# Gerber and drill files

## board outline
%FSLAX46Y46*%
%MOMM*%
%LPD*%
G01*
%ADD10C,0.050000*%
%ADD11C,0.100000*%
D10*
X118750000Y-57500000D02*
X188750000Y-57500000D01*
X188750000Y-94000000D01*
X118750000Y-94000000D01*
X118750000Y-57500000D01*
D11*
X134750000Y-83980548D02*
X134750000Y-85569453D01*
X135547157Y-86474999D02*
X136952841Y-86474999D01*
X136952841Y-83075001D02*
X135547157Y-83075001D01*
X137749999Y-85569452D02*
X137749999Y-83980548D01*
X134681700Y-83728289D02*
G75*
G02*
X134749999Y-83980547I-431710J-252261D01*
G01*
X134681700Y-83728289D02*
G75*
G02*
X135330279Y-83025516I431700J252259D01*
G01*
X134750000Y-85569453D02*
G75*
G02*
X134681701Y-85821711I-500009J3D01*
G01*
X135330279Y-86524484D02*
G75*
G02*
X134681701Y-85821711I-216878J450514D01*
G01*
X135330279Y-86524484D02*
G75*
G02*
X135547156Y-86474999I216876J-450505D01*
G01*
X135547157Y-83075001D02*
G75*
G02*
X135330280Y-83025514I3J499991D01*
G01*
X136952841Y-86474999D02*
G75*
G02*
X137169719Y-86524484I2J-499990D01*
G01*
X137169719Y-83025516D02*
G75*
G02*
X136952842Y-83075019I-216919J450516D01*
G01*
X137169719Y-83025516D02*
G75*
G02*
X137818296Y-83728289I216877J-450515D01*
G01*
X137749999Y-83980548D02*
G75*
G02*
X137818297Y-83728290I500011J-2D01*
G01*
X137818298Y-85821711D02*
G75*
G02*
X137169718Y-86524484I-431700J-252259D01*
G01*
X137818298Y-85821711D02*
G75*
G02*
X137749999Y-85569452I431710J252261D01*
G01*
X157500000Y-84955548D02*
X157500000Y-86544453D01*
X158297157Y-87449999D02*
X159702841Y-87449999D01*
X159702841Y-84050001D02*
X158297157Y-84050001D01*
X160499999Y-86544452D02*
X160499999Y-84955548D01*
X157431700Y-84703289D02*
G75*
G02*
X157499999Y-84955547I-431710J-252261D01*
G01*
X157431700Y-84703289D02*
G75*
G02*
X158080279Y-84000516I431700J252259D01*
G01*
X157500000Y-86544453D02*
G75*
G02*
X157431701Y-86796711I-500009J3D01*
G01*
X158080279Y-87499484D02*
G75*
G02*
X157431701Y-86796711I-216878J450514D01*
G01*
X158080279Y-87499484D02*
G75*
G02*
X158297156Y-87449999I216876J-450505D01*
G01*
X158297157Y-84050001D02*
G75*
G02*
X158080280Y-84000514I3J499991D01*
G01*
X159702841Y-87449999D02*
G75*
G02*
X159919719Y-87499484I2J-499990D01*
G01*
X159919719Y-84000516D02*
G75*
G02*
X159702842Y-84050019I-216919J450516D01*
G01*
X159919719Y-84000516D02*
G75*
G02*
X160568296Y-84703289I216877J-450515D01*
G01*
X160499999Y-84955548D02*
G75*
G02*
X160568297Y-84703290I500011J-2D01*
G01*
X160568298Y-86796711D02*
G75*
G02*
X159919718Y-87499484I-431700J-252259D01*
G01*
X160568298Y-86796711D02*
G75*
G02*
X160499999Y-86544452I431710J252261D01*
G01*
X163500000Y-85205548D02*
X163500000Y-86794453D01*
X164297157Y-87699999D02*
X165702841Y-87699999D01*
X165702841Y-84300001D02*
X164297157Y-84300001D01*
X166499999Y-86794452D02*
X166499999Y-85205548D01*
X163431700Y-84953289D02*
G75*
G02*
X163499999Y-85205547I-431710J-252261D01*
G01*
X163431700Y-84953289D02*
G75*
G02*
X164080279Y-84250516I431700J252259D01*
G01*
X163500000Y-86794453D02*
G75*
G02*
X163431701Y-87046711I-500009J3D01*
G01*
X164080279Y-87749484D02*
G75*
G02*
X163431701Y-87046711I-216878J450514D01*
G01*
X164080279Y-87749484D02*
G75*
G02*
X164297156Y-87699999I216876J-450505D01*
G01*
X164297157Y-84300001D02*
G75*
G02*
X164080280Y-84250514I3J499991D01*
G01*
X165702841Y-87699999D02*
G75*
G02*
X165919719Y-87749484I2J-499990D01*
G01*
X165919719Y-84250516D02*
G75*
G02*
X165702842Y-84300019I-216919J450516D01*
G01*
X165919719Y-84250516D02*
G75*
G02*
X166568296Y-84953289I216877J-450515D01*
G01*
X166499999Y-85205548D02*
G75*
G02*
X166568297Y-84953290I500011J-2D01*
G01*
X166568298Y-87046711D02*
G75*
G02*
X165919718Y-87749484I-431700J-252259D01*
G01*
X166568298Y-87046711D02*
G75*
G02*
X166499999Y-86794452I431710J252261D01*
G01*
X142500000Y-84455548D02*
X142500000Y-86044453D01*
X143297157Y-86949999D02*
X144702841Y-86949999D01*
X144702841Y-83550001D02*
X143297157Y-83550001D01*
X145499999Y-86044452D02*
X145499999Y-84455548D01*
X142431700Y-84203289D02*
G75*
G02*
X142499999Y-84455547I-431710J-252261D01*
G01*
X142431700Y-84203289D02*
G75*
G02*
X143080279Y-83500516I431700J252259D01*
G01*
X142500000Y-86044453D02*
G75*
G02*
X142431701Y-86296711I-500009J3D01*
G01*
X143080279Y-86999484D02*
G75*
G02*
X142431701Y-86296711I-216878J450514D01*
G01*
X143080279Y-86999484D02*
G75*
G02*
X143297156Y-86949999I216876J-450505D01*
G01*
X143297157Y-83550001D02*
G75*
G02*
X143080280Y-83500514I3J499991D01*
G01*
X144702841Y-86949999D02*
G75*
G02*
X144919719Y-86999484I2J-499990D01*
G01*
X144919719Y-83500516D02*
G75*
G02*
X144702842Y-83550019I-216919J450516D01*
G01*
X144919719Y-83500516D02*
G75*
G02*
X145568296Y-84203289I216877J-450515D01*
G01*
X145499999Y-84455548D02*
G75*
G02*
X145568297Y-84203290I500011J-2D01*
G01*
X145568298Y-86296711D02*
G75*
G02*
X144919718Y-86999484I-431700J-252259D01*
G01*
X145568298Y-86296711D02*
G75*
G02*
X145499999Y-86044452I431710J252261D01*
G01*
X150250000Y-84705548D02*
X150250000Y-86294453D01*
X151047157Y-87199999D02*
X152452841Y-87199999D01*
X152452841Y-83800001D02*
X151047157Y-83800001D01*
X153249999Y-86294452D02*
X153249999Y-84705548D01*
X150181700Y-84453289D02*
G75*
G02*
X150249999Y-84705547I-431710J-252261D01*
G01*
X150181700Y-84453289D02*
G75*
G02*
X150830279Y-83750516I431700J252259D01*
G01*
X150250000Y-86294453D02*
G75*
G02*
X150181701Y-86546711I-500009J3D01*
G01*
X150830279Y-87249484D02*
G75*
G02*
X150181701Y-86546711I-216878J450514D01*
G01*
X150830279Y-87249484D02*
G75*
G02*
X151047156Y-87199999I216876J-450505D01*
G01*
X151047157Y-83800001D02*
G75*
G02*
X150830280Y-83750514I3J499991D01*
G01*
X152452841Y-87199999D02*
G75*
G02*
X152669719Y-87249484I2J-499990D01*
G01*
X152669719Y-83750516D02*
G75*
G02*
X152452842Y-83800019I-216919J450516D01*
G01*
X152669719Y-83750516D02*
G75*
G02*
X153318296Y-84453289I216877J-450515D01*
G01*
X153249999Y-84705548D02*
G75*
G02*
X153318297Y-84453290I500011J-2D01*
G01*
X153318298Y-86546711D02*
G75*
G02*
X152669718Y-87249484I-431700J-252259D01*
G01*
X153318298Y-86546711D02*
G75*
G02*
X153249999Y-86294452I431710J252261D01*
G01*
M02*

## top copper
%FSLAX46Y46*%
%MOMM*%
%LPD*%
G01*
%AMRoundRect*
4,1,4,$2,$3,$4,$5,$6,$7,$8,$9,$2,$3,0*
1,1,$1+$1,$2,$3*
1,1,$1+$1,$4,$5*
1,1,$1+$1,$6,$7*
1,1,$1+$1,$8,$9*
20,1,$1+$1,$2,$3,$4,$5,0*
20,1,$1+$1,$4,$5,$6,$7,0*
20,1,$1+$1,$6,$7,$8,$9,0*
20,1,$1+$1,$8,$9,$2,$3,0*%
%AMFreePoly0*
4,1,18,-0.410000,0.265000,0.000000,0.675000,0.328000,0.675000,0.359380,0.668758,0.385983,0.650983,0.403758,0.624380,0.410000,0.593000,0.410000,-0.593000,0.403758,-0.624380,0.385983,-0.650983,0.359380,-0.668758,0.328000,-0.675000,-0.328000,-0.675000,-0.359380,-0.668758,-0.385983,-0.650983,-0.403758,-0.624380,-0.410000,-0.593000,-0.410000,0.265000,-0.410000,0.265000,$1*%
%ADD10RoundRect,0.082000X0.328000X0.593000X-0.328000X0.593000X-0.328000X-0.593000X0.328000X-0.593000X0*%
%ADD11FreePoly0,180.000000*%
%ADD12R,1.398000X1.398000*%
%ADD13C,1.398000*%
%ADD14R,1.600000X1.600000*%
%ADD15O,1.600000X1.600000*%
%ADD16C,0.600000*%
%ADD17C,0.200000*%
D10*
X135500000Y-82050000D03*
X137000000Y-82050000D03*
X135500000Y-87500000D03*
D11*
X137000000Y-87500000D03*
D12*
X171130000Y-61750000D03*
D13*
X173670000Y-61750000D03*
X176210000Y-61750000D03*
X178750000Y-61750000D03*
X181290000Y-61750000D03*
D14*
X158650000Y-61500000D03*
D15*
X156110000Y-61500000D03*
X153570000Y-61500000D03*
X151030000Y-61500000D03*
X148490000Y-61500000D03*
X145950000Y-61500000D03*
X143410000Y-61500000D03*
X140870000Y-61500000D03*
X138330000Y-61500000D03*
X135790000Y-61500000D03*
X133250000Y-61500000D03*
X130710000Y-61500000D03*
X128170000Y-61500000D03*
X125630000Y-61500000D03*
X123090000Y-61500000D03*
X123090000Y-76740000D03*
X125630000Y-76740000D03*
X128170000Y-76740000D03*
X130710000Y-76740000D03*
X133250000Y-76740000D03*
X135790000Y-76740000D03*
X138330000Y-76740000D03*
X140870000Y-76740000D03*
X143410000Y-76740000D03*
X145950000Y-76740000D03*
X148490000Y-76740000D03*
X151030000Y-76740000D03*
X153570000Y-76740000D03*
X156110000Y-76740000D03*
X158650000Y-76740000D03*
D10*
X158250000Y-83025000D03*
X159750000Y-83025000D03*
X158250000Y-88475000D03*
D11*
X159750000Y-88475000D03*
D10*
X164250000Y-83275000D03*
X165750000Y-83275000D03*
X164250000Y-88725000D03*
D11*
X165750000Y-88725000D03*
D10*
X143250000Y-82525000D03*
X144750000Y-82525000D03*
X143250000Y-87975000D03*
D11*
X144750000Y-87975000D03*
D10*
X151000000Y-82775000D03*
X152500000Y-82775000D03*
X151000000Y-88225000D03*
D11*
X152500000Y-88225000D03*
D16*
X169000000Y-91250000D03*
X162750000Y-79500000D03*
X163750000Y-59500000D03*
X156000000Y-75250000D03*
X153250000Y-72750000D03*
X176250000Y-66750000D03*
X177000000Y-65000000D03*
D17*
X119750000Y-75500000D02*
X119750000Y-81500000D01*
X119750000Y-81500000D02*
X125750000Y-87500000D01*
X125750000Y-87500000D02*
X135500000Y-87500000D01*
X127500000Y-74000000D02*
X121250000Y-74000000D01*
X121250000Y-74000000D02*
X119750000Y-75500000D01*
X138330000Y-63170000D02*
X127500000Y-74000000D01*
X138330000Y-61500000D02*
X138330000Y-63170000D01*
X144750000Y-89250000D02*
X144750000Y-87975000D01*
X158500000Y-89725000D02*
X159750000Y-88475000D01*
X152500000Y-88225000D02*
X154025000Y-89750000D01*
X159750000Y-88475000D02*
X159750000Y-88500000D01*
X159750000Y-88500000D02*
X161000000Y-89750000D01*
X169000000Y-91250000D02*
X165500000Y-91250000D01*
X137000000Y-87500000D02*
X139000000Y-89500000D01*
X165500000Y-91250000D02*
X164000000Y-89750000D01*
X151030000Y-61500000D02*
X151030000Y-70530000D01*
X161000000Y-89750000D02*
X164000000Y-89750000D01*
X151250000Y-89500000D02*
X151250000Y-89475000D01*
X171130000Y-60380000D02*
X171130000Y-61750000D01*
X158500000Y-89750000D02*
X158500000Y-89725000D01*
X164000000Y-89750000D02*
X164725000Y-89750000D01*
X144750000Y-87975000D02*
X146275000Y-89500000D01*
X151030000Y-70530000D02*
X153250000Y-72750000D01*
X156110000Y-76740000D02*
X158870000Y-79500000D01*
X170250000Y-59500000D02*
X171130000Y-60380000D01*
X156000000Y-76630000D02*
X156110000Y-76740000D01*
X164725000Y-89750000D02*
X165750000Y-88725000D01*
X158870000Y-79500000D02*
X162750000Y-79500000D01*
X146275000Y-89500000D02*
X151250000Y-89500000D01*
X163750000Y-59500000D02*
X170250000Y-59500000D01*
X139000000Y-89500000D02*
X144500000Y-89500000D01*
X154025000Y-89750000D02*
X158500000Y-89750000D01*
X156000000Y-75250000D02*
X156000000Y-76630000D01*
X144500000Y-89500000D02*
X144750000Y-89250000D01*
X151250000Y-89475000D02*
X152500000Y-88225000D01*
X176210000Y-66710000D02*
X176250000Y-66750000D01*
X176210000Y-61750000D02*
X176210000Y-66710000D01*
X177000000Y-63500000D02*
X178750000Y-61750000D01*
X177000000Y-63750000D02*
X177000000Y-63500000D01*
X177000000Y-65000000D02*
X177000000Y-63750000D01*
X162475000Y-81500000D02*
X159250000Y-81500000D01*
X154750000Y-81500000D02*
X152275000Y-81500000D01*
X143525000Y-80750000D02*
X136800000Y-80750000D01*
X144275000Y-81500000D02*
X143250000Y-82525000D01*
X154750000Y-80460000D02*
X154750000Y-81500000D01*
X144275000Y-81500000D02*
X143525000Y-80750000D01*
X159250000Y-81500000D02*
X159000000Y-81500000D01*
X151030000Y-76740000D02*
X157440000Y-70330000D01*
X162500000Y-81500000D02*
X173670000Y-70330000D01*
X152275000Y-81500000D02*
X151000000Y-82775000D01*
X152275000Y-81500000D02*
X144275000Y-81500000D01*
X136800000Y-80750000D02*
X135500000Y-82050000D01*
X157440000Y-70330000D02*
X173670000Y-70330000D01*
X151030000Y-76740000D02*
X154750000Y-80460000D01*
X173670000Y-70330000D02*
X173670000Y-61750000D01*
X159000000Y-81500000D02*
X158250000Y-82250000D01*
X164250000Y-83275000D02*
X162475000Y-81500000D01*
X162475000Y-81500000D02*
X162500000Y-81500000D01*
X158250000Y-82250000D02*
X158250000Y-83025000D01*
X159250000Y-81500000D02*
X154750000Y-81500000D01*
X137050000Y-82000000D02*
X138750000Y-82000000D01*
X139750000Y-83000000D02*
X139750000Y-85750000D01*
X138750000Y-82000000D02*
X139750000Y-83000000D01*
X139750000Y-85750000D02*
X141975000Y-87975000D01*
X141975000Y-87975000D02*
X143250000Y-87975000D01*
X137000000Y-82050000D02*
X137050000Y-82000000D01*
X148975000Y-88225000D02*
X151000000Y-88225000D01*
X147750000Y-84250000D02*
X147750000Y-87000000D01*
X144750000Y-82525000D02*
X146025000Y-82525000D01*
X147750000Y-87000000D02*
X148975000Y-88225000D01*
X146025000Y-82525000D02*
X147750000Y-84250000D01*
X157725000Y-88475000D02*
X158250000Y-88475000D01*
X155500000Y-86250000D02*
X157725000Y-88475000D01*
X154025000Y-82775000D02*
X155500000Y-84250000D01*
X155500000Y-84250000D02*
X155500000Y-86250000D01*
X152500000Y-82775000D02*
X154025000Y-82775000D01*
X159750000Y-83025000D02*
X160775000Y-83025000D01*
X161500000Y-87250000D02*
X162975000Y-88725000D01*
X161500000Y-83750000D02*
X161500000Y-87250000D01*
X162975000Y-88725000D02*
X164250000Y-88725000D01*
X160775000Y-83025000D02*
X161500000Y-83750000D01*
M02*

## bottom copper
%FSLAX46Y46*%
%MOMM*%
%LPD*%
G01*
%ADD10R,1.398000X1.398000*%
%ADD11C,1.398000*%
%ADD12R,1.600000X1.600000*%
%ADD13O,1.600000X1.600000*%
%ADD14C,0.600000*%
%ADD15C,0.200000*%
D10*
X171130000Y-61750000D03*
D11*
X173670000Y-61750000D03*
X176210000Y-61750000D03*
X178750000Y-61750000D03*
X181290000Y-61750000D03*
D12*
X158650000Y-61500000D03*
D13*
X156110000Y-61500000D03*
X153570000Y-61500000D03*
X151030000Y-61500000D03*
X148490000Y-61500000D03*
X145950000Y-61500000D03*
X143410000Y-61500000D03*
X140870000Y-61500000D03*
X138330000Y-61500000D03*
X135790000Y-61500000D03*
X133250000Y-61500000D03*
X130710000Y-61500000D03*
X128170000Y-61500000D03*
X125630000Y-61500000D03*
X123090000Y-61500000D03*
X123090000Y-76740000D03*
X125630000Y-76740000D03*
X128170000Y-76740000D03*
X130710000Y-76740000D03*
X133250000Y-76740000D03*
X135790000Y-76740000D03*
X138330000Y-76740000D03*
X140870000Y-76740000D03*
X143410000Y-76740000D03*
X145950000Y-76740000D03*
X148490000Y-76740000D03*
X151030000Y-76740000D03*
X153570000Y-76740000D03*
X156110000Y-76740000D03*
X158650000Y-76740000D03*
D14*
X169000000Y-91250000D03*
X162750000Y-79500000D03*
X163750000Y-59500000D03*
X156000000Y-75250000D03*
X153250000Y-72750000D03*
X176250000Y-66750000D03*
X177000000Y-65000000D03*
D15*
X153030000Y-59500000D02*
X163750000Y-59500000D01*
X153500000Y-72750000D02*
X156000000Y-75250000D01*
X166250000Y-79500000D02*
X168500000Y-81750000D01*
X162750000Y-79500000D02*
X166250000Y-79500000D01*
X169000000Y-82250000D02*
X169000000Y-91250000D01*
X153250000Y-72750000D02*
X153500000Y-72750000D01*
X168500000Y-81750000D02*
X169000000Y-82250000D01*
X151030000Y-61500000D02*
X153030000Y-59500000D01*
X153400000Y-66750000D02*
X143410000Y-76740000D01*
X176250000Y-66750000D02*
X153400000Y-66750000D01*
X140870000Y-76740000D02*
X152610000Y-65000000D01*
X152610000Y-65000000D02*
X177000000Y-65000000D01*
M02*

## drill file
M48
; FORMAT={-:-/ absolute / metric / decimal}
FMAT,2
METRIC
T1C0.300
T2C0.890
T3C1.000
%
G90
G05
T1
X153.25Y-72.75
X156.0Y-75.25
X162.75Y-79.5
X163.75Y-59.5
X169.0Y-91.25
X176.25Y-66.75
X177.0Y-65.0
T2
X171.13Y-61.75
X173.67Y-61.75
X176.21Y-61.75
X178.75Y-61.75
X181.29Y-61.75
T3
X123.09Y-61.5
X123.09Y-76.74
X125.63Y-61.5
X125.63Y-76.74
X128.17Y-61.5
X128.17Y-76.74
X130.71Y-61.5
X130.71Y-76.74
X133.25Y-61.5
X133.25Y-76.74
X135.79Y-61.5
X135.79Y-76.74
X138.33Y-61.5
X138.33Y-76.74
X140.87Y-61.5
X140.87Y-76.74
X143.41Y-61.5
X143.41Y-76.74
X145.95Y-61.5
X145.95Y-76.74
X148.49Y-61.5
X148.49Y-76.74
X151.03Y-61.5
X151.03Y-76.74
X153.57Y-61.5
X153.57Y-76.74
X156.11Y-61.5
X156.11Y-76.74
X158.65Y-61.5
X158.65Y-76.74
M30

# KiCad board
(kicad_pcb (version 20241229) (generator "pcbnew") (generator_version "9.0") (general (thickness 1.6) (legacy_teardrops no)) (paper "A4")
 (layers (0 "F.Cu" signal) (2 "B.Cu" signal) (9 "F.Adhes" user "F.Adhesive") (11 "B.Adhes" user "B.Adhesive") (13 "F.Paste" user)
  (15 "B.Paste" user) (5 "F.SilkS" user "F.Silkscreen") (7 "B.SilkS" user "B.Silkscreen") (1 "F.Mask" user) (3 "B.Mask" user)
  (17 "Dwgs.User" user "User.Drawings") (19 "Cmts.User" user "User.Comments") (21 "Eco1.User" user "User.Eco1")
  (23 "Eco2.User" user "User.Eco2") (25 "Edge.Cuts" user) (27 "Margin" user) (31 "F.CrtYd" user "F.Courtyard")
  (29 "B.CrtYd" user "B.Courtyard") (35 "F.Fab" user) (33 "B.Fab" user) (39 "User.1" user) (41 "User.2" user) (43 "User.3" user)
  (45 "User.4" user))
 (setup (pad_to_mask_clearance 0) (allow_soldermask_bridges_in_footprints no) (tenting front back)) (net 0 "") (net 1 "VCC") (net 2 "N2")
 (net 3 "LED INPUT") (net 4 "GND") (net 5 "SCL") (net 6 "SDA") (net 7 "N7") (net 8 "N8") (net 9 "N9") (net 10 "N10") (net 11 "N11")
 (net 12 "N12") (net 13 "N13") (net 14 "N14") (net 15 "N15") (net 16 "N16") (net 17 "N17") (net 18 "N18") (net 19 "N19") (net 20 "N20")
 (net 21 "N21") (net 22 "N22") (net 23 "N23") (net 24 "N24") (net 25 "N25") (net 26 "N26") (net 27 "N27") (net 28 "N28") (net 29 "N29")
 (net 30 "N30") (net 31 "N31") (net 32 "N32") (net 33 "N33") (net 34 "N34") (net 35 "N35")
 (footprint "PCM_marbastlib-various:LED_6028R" (layer "F.Cu") (at 136.25 84.775 90)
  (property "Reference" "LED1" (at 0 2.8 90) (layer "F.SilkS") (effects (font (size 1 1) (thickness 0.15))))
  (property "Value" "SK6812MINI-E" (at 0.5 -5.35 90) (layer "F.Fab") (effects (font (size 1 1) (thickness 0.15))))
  (fp_line (start 0.794452 -1.5) (end -0.794453 -1.5) (stroke (width 0.1) (type solid)) (layer "Edge.Cuts"))
  (fp_line (start -1.699999 -0.702843) (end -1.699999 0.702841) (stroke (width 0.1) (type solid)) (layer "Edge.Cuts"))
  (fp_line (start 1.699999 0.702841) (end 1.699999 -0.702843) (stroke (width 0.1) (type solid)) (layer "Edge.Cuts"))
  (fp_line (start -0.794452 1.499999) (end 0.794452 1.499999) (stroke (width 0.1) (type solid)) (layer "Edge.Cuts"))
  (fp_arc (start 1.046711 -1.5683) (mid 0.925123 -1.517378) (end 0.794453 -1.500001) (stroke (width 0.1) (type solid)) (layer "Edge.Cuts"))
  (fp_arc (start 1.046711 -1.5683) (mid 1.638071 -1.504036) (end 1.749484 -0.919721) (stroke (width 0.1) (type solid)) (layer "Edge.Cuts"))
  (fp_arc (start -0.794453 -1.5) (mid -0.925123 -1.517377) (end -1.046711 -1.568299) (stroke (width 0.1) (type solid)) (layer "Edge.Cuts"))
  (fp_arc (start -1.749484 -0.919721) (mid -1.638071 -1.504036) (end -1.046711 -1.568299) (stroke (width 0.1) (type solid))
   (layer "Edge.Cuts"))
  (fp_arc (start -1.749484 -0.919721) (mid -1.712527 -0.814069) (end -1.699999 -0.702844) (stroke (width 0.1) (type solid))
   (layer "Edge.Cuts"))
  (fp_arc (start 1.699999 -0.702843) (mid 1.712527 -0.814069) (end 1.749484 -0.919721) (stroke (width 0.1) (type solid)) (layer "Edge.Cuts"))
  (fp_arc (start -1.699999 0.702841) (mid -1.712527 0.814067) (end -1.749484 0.919719) (stroke (width 0.1) (type solid)) (layer "Edge.Cuts"))
  (fp_arc (start 1.749484 0.919719) (mid 1.712527 0.814067) (end 1.699999 0.702842) (stroke (width 0.1) (type solid)) (layer "Edge.Cuts"))
  (fp_arc (start 1.749484 0.919719) (mid 1.63807 1.504033) (end 1.046711 1.568296) (stroke (width 0.1) (type solid)) (layer "Edge.Cuts"))
  (fp_arc (start 0.794452 1.499999) (mid 0.925122 1.517376) (end 1.04671 1.568298) (stroke (width 0.1) (type solid)) (layer "Edge.Cuts"))
  (fp_arc (start -1.046711 1.568298) (mid -1.638072 1.504034) (end -1.749484 0.919718) (stroke (width 0.1) (type solid)) (layer "Edge.Cuts"))
  (fp_arc (start -1.046711 1.568298) (mid -0.925123 1.517376) (end -0.794452 1.499999) (stroke (width 0.1) (type solid)) (layer "Edge.Cuts"))
  (pad "1" smd roundrect (at 2.725 -0.75 180) (size 0.82 1.35) (layers "F.Cu" "F.Mask" "F.Paste") (roundrect_rratio 0.1) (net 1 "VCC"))
  (pad "2" smd roundrect (at 2.725 0.75 180) (size 0.82 1.35) (layers "F.Cu" "F.Mask" "F.Paste") (roundrect_rratio 0.1) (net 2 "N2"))
  (pad "3" smd roundrect (at -2.725 -0.75 180) (size 0.82 1.35) (layers "F.Cu" "F.Mask" "F.Paste") (roundrect_rratio 0.1)
   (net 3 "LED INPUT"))
  (pad "4" smd roundrect (at -2.725 0.75 180) (size 0.82 1.35) (layers "F.Cu" "F.Mask" "F.Paste") (roundrect_rratio 0.1) (chamfer_ratio 0.5)
   (chamfer top_left) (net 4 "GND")))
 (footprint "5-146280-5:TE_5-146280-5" (layer "F.Cu") (at 176.21 61.75)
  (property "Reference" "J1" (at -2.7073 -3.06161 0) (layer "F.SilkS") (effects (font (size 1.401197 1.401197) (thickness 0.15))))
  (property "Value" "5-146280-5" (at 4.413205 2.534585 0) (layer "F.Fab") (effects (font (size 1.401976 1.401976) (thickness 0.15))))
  (pad "1" thru_hole rect (at -5.08 0) (size 1.398 1.398) (drill 0.89) (layers "*.Cu" "*.Mask") (remove_unused_layers no) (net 4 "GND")
   (solder_mask_margin 0.102))
  (pad "2" thru_hole circle (at -2.54 0) (size 1.398 1.398) (drill 0.89) (layers "*.Cu" "*.Mask") (remove_unused_layers no) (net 1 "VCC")
   (solder_mask_margin 0.102))
  (pad "3" thru_hole circle (at 0 0) (size 1.398 1.398) (drill 0.89) (layers "*.Cu" "*.Mask") (remove_unused_layers no) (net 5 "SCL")
   (solder_mask_margin 0.102))
  (pad "4" thru_hole circle (at 2.54 0) (size 1.398 1.398) (drill 0.89) (layers "*.Cu" "*.Mask") (remove_unused_layers no) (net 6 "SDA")
   (solder_mask_margin 0.102))
  (pad "5" thru_hole circle (at 5.08 0) (size 1.398 1.398) (drill 0.89) (layers "*.Cu" "*.Mask") (remove_unused_layers no) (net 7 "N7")
   (solder_mask_margin 0.102)))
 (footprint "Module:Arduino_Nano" (layer "F.Cu") (at 158.65 61.5 -90)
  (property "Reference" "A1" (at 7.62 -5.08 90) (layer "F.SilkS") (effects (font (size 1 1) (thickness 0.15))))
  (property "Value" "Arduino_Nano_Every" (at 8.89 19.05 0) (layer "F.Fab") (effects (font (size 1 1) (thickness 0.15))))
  (pad "1" thru_hole rect (at 0 0 270) (size 1.6 1.6) (drill 1) (layers "*.Cu" "*.Mask") (remove_unused_layers no) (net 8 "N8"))
  (pad "2" thru_hole oval (at 0 2.54 270) (size 1.6 1.6) (drill 1) (layers "*.Cu" "*.Mask") (remove_unused_layers no) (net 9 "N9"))
  (pad "3" thru_hole oval (at 0 5.08 270) (size 1.6 1.6) (drill 1) (layers "*.Cu" "*.Mask") (remove_unused_layers no) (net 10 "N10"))
  (pad "4" thru_hole oval (at 0 7.62 270) (size 1.6 1.6) (drill 1) (layers "*.Cu" "*.Mask") (remove_unused_layers no) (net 4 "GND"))
  (pad "5" thru_hole oval (at 0 10.16 270) (size 1.6 1.6) (drill 1) (layers "*.Cu" "*.Mask") (remove_unused_layers no) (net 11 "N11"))
  (pad "6" thru_hole oval (at 0 12.7 270) (size 1.6 1.6) (drill 1) (layers "*.Cu" "*.Mask") (remove_unused_layers no) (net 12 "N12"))
  (pad "7" thru_hole oval (at 0 15.24 270) (size 1.6 1.6) (drill 1) (layers "*.Cu" "*.Mask") (remove_unused_layers no) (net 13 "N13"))
  (pad "8" thru_hole oval (at 0 17.78 270) (size 1.6 1.6) (drill 1) (layers "*.Cu" "*.Mask") (remove_unused_layers no) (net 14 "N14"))
  (pad "9" thru_hole oval (at 0 20.32 270) (size 1.6 1.6) (drill 1) (layers "*.Cu" "*.Mask") (remove_unused_layers no) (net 3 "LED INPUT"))
  (pad "10" thru_hole oval (at 0 22.86 270) (size 1.6 1.6) (drill 1) (layers "*.Cu" "*.Mask") (remove_unused_layers no) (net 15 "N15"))
  (pad "11" thru_hole oval (at 0 25.4 270) (size 1.6 1.6) (drill 1) (layers "*.Cu" "*.Mask") (remove_unused_layers no) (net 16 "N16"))
  (pad "12" thru_hole oval (at 0 27.94 270) (size 1.6 1.6) (drill 1) (layers "*.Cu" "*.Mask") (remove_unused_layers no) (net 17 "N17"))
  (pad "13" thru_hole oval (at 0 30.48 270) (size 1.6 1.6) (drill 1) (layers "*.Cu" "*.Mask") (remove_unused_layers no) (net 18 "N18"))
  (pad "14" thru_hole oval (at 0 33.02 270) (size 1.6 1.6) (drill 1) (layers "*.Cu" "*.Mask") (remove_unused_layers no) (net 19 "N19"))
  (pad "15" thru_hole oval (at 0 35.56 270) (size 1.6 1.6) (drill 1) (layers "*.Cu" "*.Mask") (remove_unused_layers no) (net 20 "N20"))
  (pad "16" thru_hole oval (at 15.24 35.56 270) (size 1.6 1.6) (drill 1) (layers "*.Cu" "*.Mask") (remove_unused_layers no) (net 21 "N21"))
  (pad "17" thru_hole oval (at 15.24 33.02 270) (size 1.6 1.6) (drill 1) (layers "*.Cu" "*.Mask") (remove_unused_layers no) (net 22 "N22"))
  (pad "18" thru_hole oval (at 15.24 30.48 270) (size 1.6 1.6) (drill 1) (layers "*.Cu" "*.Mask") (remove_unused_layers no) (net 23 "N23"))
  (pad "19" thru_hole oval (at 15.24 27.94 270) (size 1.6 1.6) (drill 1) (layers "*.Cu" "*.Mask") (remove_unused_layers no) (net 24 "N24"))
  (pad "20" thru_hole oval (at 15.24 25.4 270) (size 1.6 1.6) (drill 1) (layers "*.Cu" "*.Mask") (remove_unused_layers no) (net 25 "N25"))
  (pad "21" thru_hole oval (at 15.24 22.86 270) (size 1.6 1.6) (drill 1) (layers "*.Cu" "*.Mask") (remove_unused_layers no) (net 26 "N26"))
  (pad "22" thru_hole oval (at 15.24 20.32 270) (size 1.6 1.6) (drill 1) (layers "*.Cu" "*.Mask") (remove_unused_layers no) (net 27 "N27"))
  (pad "23" thru_hole oval (at 15.24 17.78 270) (size 1.6 1.6) (drill 1) (layers "*.Cu" "*.Mask") (remove_unused_layers no) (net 6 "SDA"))
  (pad "24" thru_hole oval (at 15.24 15.24 270) (size 1.6 1.6) (drill 1) (layers "*.Cu" "*.Mask") (remove_unused_layers no) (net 5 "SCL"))
  (pad "25" thru_hole oval (at 15.24 12.7 270) (size 1.6 1.6) (drill 1) (layers "*.Cu" "*.Mask") (remove_unused_layers no) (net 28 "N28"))
  (pad "26" thru_hole oval (at 15.24 10.16 270) (size 1.6 1.6) (drill 1) (layers "*.Cu" "*.Mask") (remove_unused_layers no) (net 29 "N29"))
  (pad "27" thru_hole oval (at 15.24 7.62 270) (size 1.6 1.6) (drill 1) (layers "*.Cu" "*.Mask") (remove_unused_layers no) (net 1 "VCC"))
  (pad "28" thru_hole oval (at 15.24 5.08 270) (size 1.6 1.6) (drill 1) (layers "*.Cu" "*.Mask") (remove_unused_layers no) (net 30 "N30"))
  (pad "29" thru_hole oval (at 15.24 2.54 270) (size 1.6 1.6) (drill 1) (layers "*.Cu" "*.Mask") (remove_unused_layers no) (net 4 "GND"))
  (pad "30" thru_hole oval (at 15.24 0 270) (size 1.6 1.6) (drill 1) (layers "*.Cu" "*.Mask") (remove_unused_layers no) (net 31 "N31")))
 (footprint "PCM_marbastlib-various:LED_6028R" (layer "F.Cu") (at 159 85.75 90)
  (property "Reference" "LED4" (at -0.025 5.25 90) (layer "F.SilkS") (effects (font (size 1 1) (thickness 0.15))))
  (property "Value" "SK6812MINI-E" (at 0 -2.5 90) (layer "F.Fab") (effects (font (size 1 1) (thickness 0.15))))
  (fp_line (start 0.794452 -1.5) (end -0.794453 -1.5) (stroke (width 0.1) (type solid)) (layer "Edge.Cuts"))
  (fp_line (start -1.699999 -0.702843) (end -1.699999 0.702841) (stroke (width 0.1) (type solid)) (layer "Edge.Cuts"))
  (fp_line (start 1.699999 0.702841) (end 1.699999 -0.702843) (stroke (width 0.1) (type solid)) (layer "Edge.Cuts"))
  (fp_line (start -0.794452 1.499999) (end 0.794452 1.499999) (stroke (width 0.1) (type solid)) (layer "Edge.Cuts"))
  (fp_arc (start 1.046711 -1.5683) (mid 0.925123 -1.517378) (end 0.794453 -1.500001) (stroke (width 0.1) (type solid)) (layer "Edge.Cuts"))
  (fp_arc (start 1.046711 -1.5683) (mid 1.638071 -1.504036) (end 1.749484 -0.919721) (stroke (width 0.1) (type solid)) (layer "Edge.Cuts"))
  (fp_arc (start -0.794453 -1.5) (mid -0.925123 -1.517377) (end -1.046711 -1.568299) (stroke (width 0.1) (type solid)) (layer "Edge.Cuts"))
  (fp_arc (start -1.749484 -0.919721) (mid -1.638071 -1.504036) (end -1.046711 -1.568299) (stroke (width 0.1) (type solid))
   (layer "Edge.Cuts"))
  (fp_arc (start -1.749484 -0.919721) (mid -1.712527 -0.814069) (end -1.699999 -0.702844) (stroke (width 0.1) (type solid))
   (layer "Edge.Cuts"))
  (fp_arc (start 1.699999 -0.702843) (mid 1.712527 -0.814069) (end 1.749484 -0.919721) (stroke (width 0.1) (type solid)) (layer "Edge.Cuts"))
  (fp_arc (start -1.699999 0.702841) (mid -1.712527 0.814067) (end -1.749484 0.919719) (stroke (width 0.1) (type solid)) (layer "Edge.Cuts"))
  (fp_arc (start 1.749484 0.919719) (mid 1.712527 0.814067) (end 1.699999 0.702842) (stroke (width 0.1) (type solid)) (layer "Edge.Cuts"))
  (fp_arc (start 1.749484 0.919719) (mid 1.63807 1.504033) (end 1.046711 1.568296) (stroke (width 0.1) (type solid)) (layer "Edge.Cuts"))
  (fp_arc (start 0.794452 1.499999) (mid 0.925122 1.517376) (end 1.04671 1.568298) (stroke (width 0.1) (type solid)) (layer "Edge.Cuts"))
  (fp_arc (start -1.046711 1.568298) (mid -1.638072 1.504034) (end -1.749484 0.919718) (stroke (width 0.1) (type solid)) (layer "Edge.Cuts"))
  (fp_arc (start -1.046711 1.568298) (mid -0.925123 1.517376) (end -0.794452 1.499999) (stroke (width 0.1) (type solid)) (layer "Edge.Cuts"))
  (pad "1" smd roundrect (at 2.725 -0.75 180) (size 0.82 1.35) (layers "F.Cu" "F.Mask" "F.Paste") (roundrect_rratio 0.1) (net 1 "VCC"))
  (pad "2" smd roundrect (at 2.725 0.75 180) (size 0.82 1.35) (layers "F.Cu" "F.Mask" "F.Paste") (roundrect_rratio 0.1) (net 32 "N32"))
  (pad "3" smd roundrect (at -2.725 -0.75 180) (size 0.82 1.35) (layers "F.Cu" "F.Mask" "F.Paste") (roundrect_rratio 0.1) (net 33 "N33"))
  (pad "4" smd roundrect (at -2.725 0.75 180) (size 0.82 1.35) (layers "F.Cu" "F.Mask" "F.Paste") (roundrect_rratio 0.1) (chamfer_ratio 0.5)
   (chamfer top_left) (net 4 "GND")))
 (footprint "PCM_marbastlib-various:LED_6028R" (layer "F.Cu") (at 165 86 90)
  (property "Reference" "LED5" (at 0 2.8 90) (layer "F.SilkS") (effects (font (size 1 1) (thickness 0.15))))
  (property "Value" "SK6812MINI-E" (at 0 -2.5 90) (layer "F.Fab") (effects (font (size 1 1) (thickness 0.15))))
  (fp_line (start 0.794452 -1.5) (end -0.794453 -1.5) (stroke (width 0.1) (type solid)) (layer "Edge.Cuts"))
  (fp_line (start -1.699999 -0.702843) (end -1.699999 0.702841) (stroke (width 0.1) (type solid)) (layer "Edge.Cuts"))
  (fp_line (start 1.699999 0.702841) (end 1.699999 -0.702843) (stroke (width 0.1) (type solid)) (layer "Edge.Cuts"))
  (fp_line (start -0.794452 1.499999) (end 0.794452 1.499999) (stroke (width 0.1) (type solid)) (layer "Edge.Cuts"))
  (fp_arc (start 1.046711 -1.5683) (mid 0.925123 -1.517378) (end 0.794453 -1.500001) (stroke (width 0.1) (type solid)) (layer "Edge.Cuts"))
  (fp_arc (start 1.046711 -1.5683) (mid 1.638071 -1.504036) (end 1.749484 -0.919721) (stroke (width 0.1) (type solid)) (layer "Edge.Cuts"))
  (fp_arc (start -0.794453 -1.5) (mid -0.925123 -1.517377) (end -1.046711 -1.568299) (stroke (width 0.1) (type solid)) (layer "Edge.Cuts"))
  (fp_arc (start -1.749484 -0.919721) (mid -1.638071 -1.504036) (end -1.046711 -1.568299) (stroke (width 0.1) (type solid))
   (layer "Edge.Cuts"))
  (fp_arc (start -1.749484 -0.919721) (mid -1.712527 -0.814069) (end -1.699999 -0.702844) (stroke (width 0.1) (type solid))
   (layer "Edge.Cuts"))
  (fp_arc (start 1.699999 -0.702843) (mid 1.712527 -0.814069) (end 1.749484 -0.919721) (stroke (width 0.1) (type solid)) (layer "Edge.Cuts"))
  (fp_arc (start -1.699999 0.702841) (mid -1.712527 0.814067) (end -1.749484 0.919719) (stroke (width 0.1) (type solid)) (layer "Edge.Cuts"))
  (fp_arc (start 1.749484 0.919719) (mid 1.712527 0.814067) (end 1.699999 0.702842) (stroke (width 0.1) (type solid)) (layer "Edge.Cuts"))
  (fp_arc (start 1.749484 0.919719) (mid 1.63807 1.504033) (end 1.046711 1.568296) (stroke (width 0.1) (type solid)) (layer "Edge.Cuts"))
  (fp_arc (start 0.794452 1.499999) (mid 0.925122 1.517376) (end 1.04671 1.568298) (stroke (width 0.1) (type solid)) (layer "Edge.Cuts"))
  (fp_arc (start -1.046711 1.568298) (mid -1.638072 1.504034) (end -1.749484 0.919718) (stroke (width 0.1) (type solid)) (layer "Edge.Cuts"))
  (fp_arc (start -1.046711 1.568298) (mid -0.925123 1.517376) (end -0.794452 1.499999) (stroke (width 0.1) (type solid)) (layer "Edge.Cuts"))
  (pad "1" smd roundrect (at 2.725 -0.75 180) (size 0.82 1.35) (layers "F.Cu" "F.Mask" "F.Paste") (roundrect_rratio 0.1) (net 1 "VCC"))
  (pad "2" smd roundrect (at 2.725 0.75 180) (size 0.82 1.35) (layers "F.Cu" "F.Mask" "F.Paste") (roundrect_rratio 0.1) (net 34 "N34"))
  (pad "3" smd roundrect (at -2.725 -0.75 180) (size 0.82 1.35) (layers "F.Cu" "F.Mask" "F.Paste") (roundrect_rratio 0.1) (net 32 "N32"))
  (pad "4" smd roundrect (at -2.725 0.75 180) (size 0.82 1.35) (layers "F.Cu" "F.Mask" "F.Paste") (roundrect_rratio 0.1) (chamfer_ratio 0.5)
   (chamfer top_left) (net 4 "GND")))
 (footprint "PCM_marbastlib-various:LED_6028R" (layer "F.Cu") (at 144 85.25 90)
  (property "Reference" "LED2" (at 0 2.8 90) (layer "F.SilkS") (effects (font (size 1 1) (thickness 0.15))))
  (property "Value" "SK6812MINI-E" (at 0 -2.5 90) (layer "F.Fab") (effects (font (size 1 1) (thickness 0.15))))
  (fp_line (start 0.794452 -1.5) (end -0.794453 -1.5) (stroke (width 0.1) (type solid)) (layer "Edge.Cuts"))
  (fp_line (start -1.699999 -0.702843) (end -1.699999 0.702841) (stroke (width 0.1) (type solid)) (layer "Edge.Cuts"))
  (fp_line (start 1.699999 0.702841) (end 1.699999 -0.702843) (stroke (width 0.1) (type solid)) (layer "Edge.Cuts"))
  (fp_line (start -0.794452 1.499999) (end 0.794452 1.499999) (stroke (width 0.1) (type solid)) (layer "Edge.Cuts"))
  (fp_arc (start 1.046711 -1.5683) (mid 0.925123 -1.517378) (end 0.794453 -1.500001) (stroke (width 0.1) (type solid)) (layer "Edge.Cuts"))
  (fp_arc (start 1.046711 -1.5683) (mid 1.638071 -1.504036) (end 1.749484 -0.919721) (stroke (width 0.1) (type solid)) (layer "Edge.Cuts"))
  (fp_arc (start -0.794453 -1.5) (mid -0.925123 -1.517377) (end -1.046711 -1.568299) (stroke (width 0.1) (type solid)) (layer "Edge.Cuts"))
  (fp_arc (start -1.749484 -0.919721) (mid -1.638071 -1.504036) (end -1.046711 -1.568299) (stroke (width 0.1) (type solid))
   (layer "Edge.Cuts"))
  (fp_arc (start -1.749484 -0.919721) (mid -1.712527 -0.814069) (end -1.699999 -0.702844) (stroke (width 0.1) (type solid))
   (layer "Edge.Cuts"))
  (fp_arc (start 1.699999 -0.702843) (mid 1.712527 -0.814069) (end 1.749484 -0.919721) (stroke (width 0.1) (type solid)) (layer "Edge.Cuts"))
  (fp_arc (start -1.699999 0.702841) (mid -1.712527 0.814067) (end -1.749484 0.919719) (stroke (width 0.1) (type solid)) (layer "Edge.Cuts"))
  (fp_arc (start 1.749484 0.919719) (mid 1.712527 0.814067) (end 1.699999 0.702842) (stroke (width 0.1) (type solid)) (layer "Edge.Cuts"))
  (fp_arc (start 1.749484 0.919719) (mid 1.63807 1.504033) (end 1.046711 1.568296) (stroke (width 0.1) (type solid)) (layer "Edge.Cuts"))
  (fp_arc (start 0.794452 1.499999) (mid 0.925122 1.517376) (end 1.04671 1.568298) (stroke (width 0.1) (type solid)) (layer "Edge.Cuts"))
  (fp_arc (start -1.046711 1.568298) (mid -1.638072 1.504034) (end -1.749484 0.919718) (stroke (width 0.1) (type solid)) (layer "Edge.Cuts"))
  (fp_arc (start -1.046711 1.568298) (mid -0.925123 1.517376) (end -0.794452 1.499999) (stroke (width 0.1) (type solid)) (layer "Edge.Cuts"))
  (pad "1" smd roundrect (at 2.725 -0.75 180) (size 0.82 1.35) (layers "F.Cu" "F.Mask" "F.Paste") (roundrect_rratio 0.1) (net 1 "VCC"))
  (pad "2" smd roundrect (at 2.725 0.75 180) (size 0.82 1.35) (layers "F.Cu" "F.Mask" "F.Paste") (roundrect_rratio 0.1) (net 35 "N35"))
  (pad "3" smd roundrect (at -2.725 -0.75 180) (size 0.82 1.35) (layers "F.Cu" "F.Mask" "F.Paste") (roundrect_rratio 0.1) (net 2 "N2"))
  (pad "4" smd roundrect (at -2.725 0.75 180) (size 0.82 1.35) (layers "F.Cu" "F.Mask" "F.Paste") (roundrect_rratio 0.1) (chamfer_ratio 0.5)
   (chamfer top_left) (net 4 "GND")))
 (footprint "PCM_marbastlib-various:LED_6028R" (layer "F.Cu") (at 151.75 85.5 90)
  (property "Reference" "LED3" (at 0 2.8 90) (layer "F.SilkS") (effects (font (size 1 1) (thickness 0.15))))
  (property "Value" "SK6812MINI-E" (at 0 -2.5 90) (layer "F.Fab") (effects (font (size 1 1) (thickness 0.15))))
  (fp_line (start 0.794452 -1.5) (end -0.794453 -1.5) (stroke (width 0.1) (type solid)) (layer "Edge.Cuts"))
  (fp_line (start -1.699999 -0.702843) (end -1.699999 0.702841) (stroke (width 0.1) (type solid)) (layer "Edge.Cuts"))
  (fp_line (start 1.699999 0.702841) (end 1.699999 -0.702843) (stroke (width 0.1) (type solid)) (layer "Edge.Cuts"))
  (fp_line (start -0.794452 1.499999) (end 0.794452 1.499999) (stroke (width 0.1) (type solid)) (layer "Edge.Cuts"))
  (fp_arc (start 1.046711 -1.5683) (mid 0.925123 -1.517378) (end 0.794453 -1.500001) (stroke (width 0.1) (type solid)) (layer "Edge.Cuts"))
  (fp_arc (start 1.046711 -1.5683) (mid 1.638071 -1.504036) (end 1.749484 -0.919721) (stroke (width 0.1) (type solid)) (layer "Edge.Cuts"))
  (fp_arc (start -0.794453 -1.5) (mid -0.925123 -1.517377) (end -1.046711 -1.568299) (stroke (width 0.1) (type solid)) (layer "Edge.Cuts"))
  (fp_arc (start -1.749484 -0.919721) (mid -1.638071 -1.504036) (end -1.046711 -1.568299) (stroke (width 0.1) (type solid))
   (layer "Edge.Cuts"))
  (fp_arc (start -1.749484 -0.919721) (mid -1.712527 -0.814069) (end -1.699999 -0.702844) (stroke (width 0.1) (type solid))
   (layer "Edge.Cuts"))
  (fp_arc (start 1.699999 -0.702843) (mid 1.712527 -0.814069) (end 1.749484 -0.919721) (stroke (width 0.1) (type solid)) (layer "Edge.Cuts"))
  (fp_arc (start -1.699999 0.702841) (mid -1.712527 0.814067) (end -1.749484 0.919719) (stroke (width 0.1) (type solid)) (layer "Edge.Cuts"))
  (fp_arc (start 1.749484 0.919719) (mid 1.712527 0.814067) (end 1.699999 0.702842) (stroke (width 0.1) (type solid)) (layer "Edge.Cuts"))
  (fp_arc (start 1.749484 0.919719) (mid 1.63807 1.504033) (end 1.046711 1.568296) (stroke (width 0.1) (type solid)) (layer "Edge.Cuts"))
  (fp_arc (start 0.794452 1.499999) (mid 0.925122 1.517376) (end 1.04671 1.568298) (stroke (width 0.1) (type solid)) (layer "Edge.Cuts"))
  (fp_arc (start -1.046711 1.568298) (mid -1.638072 1.504034) (end -1.749484 0.919718) (stroke (width 0.1) (type solid)) (layer "Edge.Cuts"))
  (fp_arc (start -1.046711 1.568298) (mid -0.925123 1.517376) (end -0.794452 1.499999) (stroke (width 0.1) (type solid)) (layer "Edge.Cuts"))
  (pad "1" smd roundrect (at 2.725 -0.75 180) (size 0.82 1.35) (layers "F.Cu" "F.Mask" "F.Paste") (roundrect_rratio 0.1) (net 1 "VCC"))
  (pad "2" smd roundrect (at 2.725 0.75 180) (size 0.82 1.35) (layers "F.Cu" "F.Mask" "F.Paste") (roundrect_rratio 0.1) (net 33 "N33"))
  (pad "3" smd roundrect (at -2.725 -0.75 180) (size 0.82 1.35) (layers "F.Cu" "F.Mask" "F.Paste") (roundrect_rratio 0.1) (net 35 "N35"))
  (pad "4" smd roundrect (at -2.725 0.75 180) (size 0.82 1.35) (layers "F.Cu" "F.Mask" "F.Paste") (roundrect_rratio 0.1) (chamfer_ratio 0.5)
   (chamfer top_left) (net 4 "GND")))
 (gr_rect (start 118.75 57.5) (end 188.75 94) (stroke (width 0.05) (type default)) (fill no) (layer "Edge.Cuts"))
 (segment (start 119.75 75.5) (end 119.75 81.5) (width 0.2) (layer "F.Cu") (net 3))
 (segment (start 119.75 81.5) (end 125.75 87.5) (width 0.2) (layer "F.Cu") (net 3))
 (segment (start 125.75 87.5) (end 135.5 87.5) (width 0.2) (layer "F.Cu") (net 3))
 (segment (start 127.5 74) (end 121.25 74) (width 0.2) (layer "F.Cu") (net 3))
 (segment (start 121.25 74) (end 119.75 75.5) (width 0.2) (layer "F.Cu") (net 3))
 (segment (start 138.33 63.17) (end 127.5 74) (width 0.2) (layer "F.Cu") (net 3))
 (segment (start 138.33 61.5) (end 138.33 63.17) (width 0.2) (layer "F.Cu") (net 3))
 (segment (start 144.75 89.25) (end 144.75 87.975) (width 0.2) (layer "F.Cu") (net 4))
 (segment (start 158.5 89.725) (end 159.75 88.475) (width 0.2) (layer "F.Cu") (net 4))
 (segment (start 152.5 88.225) (end 154.025 89.75) (width 0.2) (layer "F.Cu") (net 4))
 (segment (start 159.75 88.475) (end 159.75 88.5) (width 0.2) (layer "F.Cu") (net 4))
 (segment (start 159.75 88.5) (end 161 89.75) (width 0.2) (layer "F.Cu") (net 4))
 (segment (start 169 91.25) (end 165.5 91.25) (width 0.2) (layer "F.Cu") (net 4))
 (segment (start 137 87.5) (end 139 89.5) (width 0.2) (layer "F.Cu") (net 4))
 (segment (start 165.5 91.25) (end 164 89.75) (width 0.2) (layer "F.Cu") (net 4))
 (segment (start 151.03 61.5) (end 151.03 70.53) (width 0.2) (layer "F.Cu") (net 4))
 (segment (start 161 89.75) (end 164 89.75) (width 0.2) (layer "F.Cu") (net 4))
 (segment (start 151.25 89.5) (end 151.25 89.475) (width 0.2) (layer "F.Cu") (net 4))
 (segment (start 171.13 60.38) (end 171.13 61.75) (width 0.2) (layer "F.Cu") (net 4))
 (segment (start 158.5 89.75) (end 158.5 89.725) (width 0.2) (layer "F.Cu") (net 4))
 (segment (start 164 89.75) (end 164.725 89.75) (width 0.2) (layer "F.Cu") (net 4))
 (segment (start 144.75 87.975) (end 146.275 89.5) (width 0.2) (layer "F.Cu") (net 4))
 (segment (start 151.03 70.53) (end 153.25 72.75) (width 0.2) (layer "F.Cu") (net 4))
 (segment (start 156.11 76.74) (end 158.87 79.5) (width 0.2) (layer "F.Cu") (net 4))
 (segment (start 170.25 59.5) (end 171.13 60.38) (width 0.2) (layer "F.Cu") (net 4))
 (segment (start 156 76.63) (end 156.11 76.74) (width 0.2) (layer "F.Cu") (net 4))
 (segment (start 164.725 89.75) (end 165.75 88.725) (width 0.2) (layer "F.Cu") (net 4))
 (segment (start 158.87 79.5) (end 162.75 79.5) (width 0.2) (layer "F.Cu") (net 4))
 (segment (start 146.275 89.5) (end 151.25 89.5) (width 0.2) (layer "F.Cu") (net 4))
 (segment (start 163.75 59.5) (end 170.25 59.5) (width 0.2) (layer "F.Cu") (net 4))
 (segment (start 139 89.5) (end 144.5 89.5) (width 0.2) (layer "F.Cu") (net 4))
 (segment (start 154.025 89.75) (end 158.5 89.75) (width 0.2) (layer "F.Cu") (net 4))
 (segment (start 156 75.25) (end 156 76.63) (width 0.2) (layer "F.Cu") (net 4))
 (segment (start 144.5 89.5) (end 144.75 89.25) (width 0.2) (layer "F.Cu") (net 4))
 (segment (start 151.25 89.475) (end 152.5 88.225) (width 0.2) (layer "F.Cu") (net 4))
 (via (at 169 91.25) (size 0.6) (drill 0.3) (layers "F.Cu" "B.Cu") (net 4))
 (via (at 162.75 79.5) (size 0.6) (drill 0.3) (layers "F.Cu" "B.Cu") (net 4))
 (via (at 163.75 59.5) (size 0.6) (drill 0.3) (layers "F.Cu" "B.Cu") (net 4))
 (via (at 156 75.25) (size 0.6) (drill 0.3) (layers "F.Cu" "B.Cu") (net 4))
 (via (at 153.25 72.75) (size 0.6) (drill 0.3) (layers "F.Cu" "B.Cu") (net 4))
 (segment (start 153.03 59.5) (end 163.75 59.5) (width 0.2) (layer "B.Cu") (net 4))
 (segment (start 153.5 72.75) (end 156 75.25) (width 0.2) (layer "B.Cu") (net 4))
 (segment (start 166.25 79.5) (end 168.5 81.75) (width 0.2) (layer "B.Cu") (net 4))
 (segment (start 162.75 79.5) (end 166.25 79.5) (width 0.2) (layer "B.Cu") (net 4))
 (segment (start 169 82.25) (end 169 91.25) (width 0.2) (layer "B.Cu") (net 4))
 (segment (start 153.25 72.75) (end 153.5 72.75) (width 0.2) (layer "B.Cu") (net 4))
 (segment (start 168.5 81.75) (end 169 82.25) (width 0.2) (layer "B.Cu") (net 4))
 (segment (start 151.03 61.5) (end 153.03 59.5) (width 0.2) (layer "B.Cu") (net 4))
 (segment (start 176.21 66.71) (end 176.25 66.75) (width 0.2) (layer "F.Cu") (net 5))
 (segment (start 176.21 61.75) (end 176.21 66.71) (width 0.2) (layer "F.Cu") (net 5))
 (via (at 176.25 66.75) (size 0.6) (drill 0.3) (layers "F.Cu" "B.Cu") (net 5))
 (segment (start 153.4 66.75) (end 143.41 76.74) (width 0.2) (layer "B.Cu") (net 5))
 (segment (start 176.25 66.75) (end 153.4 66.75) (width 0.2) (layer "B.Cu") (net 5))
 (segment (start 177 63.5) (end 178.75 61.75) (width 0.2) (layer "F.Cu") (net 6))
 (segment (start 177 63.75) (end 177 63.5) (width 0.2) (layer "F.Cu") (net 6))
 (segment (start 177 65) (end 177 63.75) (width 0.2) (layer "F.Cu") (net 6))
 (via (at 177 65) (size 0.6) (drill 0.3) (layers "F.Cu" "B.Cu") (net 6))
 (segment (start 140.87 76.74) (end 152.61 65) (width 0.2) (layer "B.Cu") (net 6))
 (segment (start 152.61 65) (end 177 65) (width 0.2) (layer "B.Cu") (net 6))
 (segment (start 162.475 81.5) (end 159.25 81.5) (width 0.2) (layer "F.Cu") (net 1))
 (segment (start 154.75 81.5) (end 152.275 81.5) (width 0.2) (layer "F.Cu") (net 1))
 (segment (start 143.525 80.75) (end 136.8 80.75) (width 0.2) (layer "F.Cu") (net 1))
 (segment (start 144.275 81.5) (end 143.25 82.525) (width 0.2) (layer "F.Cu") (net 1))
 (segment (start 154.75 80.46) (end 154.75 81.5) (width 0.2) (layer "F.Cu") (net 1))
 (segment (start 144.275 81.5) (end 143.525 80.75) (width 0.2) (layer "F.Cu") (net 1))
 (segment (start 159.25 81.5) (end 159 81.5) (width 0.2) (layer "F.Cu") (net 1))
 (segment (start 151.03 76.74) (end 157.44 70.33) (width 0.2) (layer "F.Cu") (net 1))
 (segment (start 162.5 81.5) (end 173.67 70.33) (width 0.2) (layer "F.Cu") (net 1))
 (segment (start 152.275 81.5) (end 151 82.775) (width 0.2) (layer "F.Cu") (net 1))
 (segment (start 152.275 81.5) (end 144.275 81.5) (width 0.2) (layer "F.Cu") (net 1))
 (segment (start 136.8 80.75) (end 135.5 82.05) (width 0.2) (layer "F.Cu") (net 1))
 (segment (start 157.44 70.33) (end 173.67 70.33) (width 0.2) (layer "F.Cu") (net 1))
 (segment (start 151.03 76.74) (end 154.75 80.46) (width 0.2) (layer "F.Cu") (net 1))
 (segment (start 173.67 70.33) (end 173.67 61.75) (width 0.2) (layer "F.Cu") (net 1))
 (segment (start 159 81.5) (end 158.25 82.25) (width 0.2) (layer "F.Cu") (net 1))
 (segment (start 164.25 83.275) (end 162.475 81.5) (width 0.2) (layer "F.Cu") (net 1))
 (segment (start 162.475 81.5) (end 162.5 81.5) (width 0.2) (layer "F.Cu") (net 1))
 (segment (start 158.25 82.25) (end 158.25 83.025) (width 0.2) (layer "F.Cu") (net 1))
 (segment (start 159.25 81.5) (end 154.75 81.5) (width 0.2) (layer "F.Cu") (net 1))
 (segment (start 137.05 82) (end 138.75 82) (width 0.2) (layer "F.Cu") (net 2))
 (segment (start 139.75 83) (end 139.75 85.75) (width 0.2) (layer "F.Cu") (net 2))
 (segment (start 138.75 82) (end 139.75 83) (width 0.2) (layer "F.Cu") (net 2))
 (segment (start 139.75 85.75) (end 141.975 87.975) (width 0.2) (layer "F.Cu") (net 2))
 (segment (start 141.975 87.975) (end 143.25 87.975) (width 0.2) (layer "F.Cu") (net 2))
 (segment (start 137 82.05) (end 137.05 82) (width 0.2) (layer "F.Cu") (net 2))
 (segment (start 148.975 88.225) (end 151 88.225) (width 0.2) (layer "F.Cu") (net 35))
 (segment (start 147.75 84.25) (end 147.75 87) (width 0.2) (layer "F.Cu") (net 35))
 (segment (start 144.75 82.525) (end 146.025 82.525) (width 0.2) (layer "F.Cu") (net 35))
 (segment (start 147.75 87) (end 148.975 88.225) (width 0.2) (layer "F.Cu") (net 35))
 (segment (start 146.025 82.525) (end 147.75 84.25) (width 0.2) (layer "F.Cu") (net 35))
 (segment (start 157.725 88.475) (end 158.25 88.475) (width 0.2) (layer "F.Cu") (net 33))
 (segment (start 155.5 86.25) (end 157.725 88.475) (width 0.2) (layer "F.Cu") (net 33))
 (segment (start 154.025 82.775) (end 155.5 84.25) (width 0.2) (layer "F.Cu") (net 33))
 (segment (start 155.5 84.25) (end 155.5 86.25) (width 0.2) (layer "F.Cu") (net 33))
 (segment (start 152.5 82.775) (end 154.025 82.775) (width 0.2) (layer "F.Cu") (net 33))
 (segment (start 159.75 83.025) (end 160.775 83.025) (width 0.2) (layer "F.Cu") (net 32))
 (segment (start 161.5 87.25) (end 162.975 88.725) (width 0.2) (layer "F.Cu") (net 32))
 (segment (start 161.5 83.75) (end 161.5 87.25) (width 0.2) (layer "F.Cu") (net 32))
 (segment (start 162.975 88.725) (end 164.25 88.725) (width 0.2) (layer "F.Cu") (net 32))
 (segment (start 160.775 83.025) (end 161.5 83.75) (width 0.2) (layer "F.Cu") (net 32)))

